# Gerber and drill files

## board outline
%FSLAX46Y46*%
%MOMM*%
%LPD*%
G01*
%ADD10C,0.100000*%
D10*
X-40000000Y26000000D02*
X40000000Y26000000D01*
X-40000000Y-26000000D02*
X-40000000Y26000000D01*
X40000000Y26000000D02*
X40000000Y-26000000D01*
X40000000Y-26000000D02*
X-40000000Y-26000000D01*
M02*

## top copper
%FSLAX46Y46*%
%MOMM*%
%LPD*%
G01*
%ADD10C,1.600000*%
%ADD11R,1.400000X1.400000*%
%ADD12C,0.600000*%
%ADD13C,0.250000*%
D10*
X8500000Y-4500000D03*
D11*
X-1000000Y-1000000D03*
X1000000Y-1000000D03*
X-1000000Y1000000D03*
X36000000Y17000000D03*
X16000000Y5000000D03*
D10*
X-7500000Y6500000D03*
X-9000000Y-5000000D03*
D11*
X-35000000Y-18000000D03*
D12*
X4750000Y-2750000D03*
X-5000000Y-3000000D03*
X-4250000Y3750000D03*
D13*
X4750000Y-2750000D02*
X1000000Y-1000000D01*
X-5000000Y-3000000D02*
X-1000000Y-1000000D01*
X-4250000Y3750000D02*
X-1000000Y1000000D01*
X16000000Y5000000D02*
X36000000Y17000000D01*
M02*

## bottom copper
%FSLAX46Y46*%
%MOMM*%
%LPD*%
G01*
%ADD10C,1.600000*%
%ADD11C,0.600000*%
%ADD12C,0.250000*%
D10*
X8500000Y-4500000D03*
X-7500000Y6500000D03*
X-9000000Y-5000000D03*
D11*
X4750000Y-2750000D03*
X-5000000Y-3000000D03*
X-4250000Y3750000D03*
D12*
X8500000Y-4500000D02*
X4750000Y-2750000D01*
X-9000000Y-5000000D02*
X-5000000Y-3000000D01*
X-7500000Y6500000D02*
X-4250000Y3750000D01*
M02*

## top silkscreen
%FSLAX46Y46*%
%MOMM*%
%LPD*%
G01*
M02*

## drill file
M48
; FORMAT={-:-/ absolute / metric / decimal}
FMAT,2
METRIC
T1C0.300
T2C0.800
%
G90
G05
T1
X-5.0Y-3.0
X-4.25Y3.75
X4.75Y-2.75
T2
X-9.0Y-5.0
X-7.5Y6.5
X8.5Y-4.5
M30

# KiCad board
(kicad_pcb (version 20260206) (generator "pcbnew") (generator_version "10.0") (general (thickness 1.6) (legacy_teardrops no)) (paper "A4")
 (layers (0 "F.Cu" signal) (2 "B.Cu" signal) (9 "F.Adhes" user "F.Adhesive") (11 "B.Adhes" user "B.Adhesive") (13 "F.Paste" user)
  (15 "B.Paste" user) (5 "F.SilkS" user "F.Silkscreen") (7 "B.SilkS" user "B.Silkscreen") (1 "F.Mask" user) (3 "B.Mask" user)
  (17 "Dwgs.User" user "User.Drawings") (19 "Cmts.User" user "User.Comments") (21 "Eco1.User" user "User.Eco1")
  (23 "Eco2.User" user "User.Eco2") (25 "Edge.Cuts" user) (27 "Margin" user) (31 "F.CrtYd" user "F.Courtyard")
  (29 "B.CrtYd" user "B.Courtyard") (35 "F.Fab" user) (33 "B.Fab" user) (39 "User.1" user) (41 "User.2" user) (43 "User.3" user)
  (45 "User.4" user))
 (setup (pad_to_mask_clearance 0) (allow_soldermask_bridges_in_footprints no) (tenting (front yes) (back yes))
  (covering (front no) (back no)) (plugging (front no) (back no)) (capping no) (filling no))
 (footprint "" (layer "F.Cu") (at 8.5 4.5)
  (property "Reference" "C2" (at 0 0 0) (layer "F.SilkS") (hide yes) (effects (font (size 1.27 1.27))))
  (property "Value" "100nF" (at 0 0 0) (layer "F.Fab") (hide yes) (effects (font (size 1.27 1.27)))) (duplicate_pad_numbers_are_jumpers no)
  (pad "1" thru_hole circle (at 0 0) (size 1.6 1.6) (drill 0.8) (layers "*.Cu" "*.Mask") (remove_unused_layers no) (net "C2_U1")))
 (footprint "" (layer "F.Cu") (at 0 0)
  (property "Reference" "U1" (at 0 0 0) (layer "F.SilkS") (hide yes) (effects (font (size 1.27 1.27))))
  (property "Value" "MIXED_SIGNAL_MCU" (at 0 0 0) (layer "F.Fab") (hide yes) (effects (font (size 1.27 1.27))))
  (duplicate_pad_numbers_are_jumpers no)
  (pad "1" smd rect (at -1 1) (size 1.4 1.4) (layers "F.Cu" "F.Mask" "F.Paste") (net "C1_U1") (thermal_bridge_angle 45))
  (pad "2" smd rect (at 1 1) (size 1.4 1.4) (layers "F.Cu" "F.Mask" "F.Paste") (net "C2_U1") (thermal_bridge_angle 45))
  (pad "3" smd rect (at -1 -1) (size 1.4 1.4) (layers "F.Cu" "F.Mask" "F.Paste") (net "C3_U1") (thermal_bridge_angle 45)))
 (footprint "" (layer "F.Cu") (at 36 -17)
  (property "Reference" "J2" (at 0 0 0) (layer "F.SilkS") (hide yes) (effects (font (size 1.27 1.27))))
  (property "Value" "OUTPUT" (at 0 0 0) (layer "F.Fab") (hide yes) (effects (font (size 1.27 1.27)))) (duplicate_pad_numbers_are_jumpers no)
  (pad "1" smd rect (at 0 0) (size 1.4 1.4) (layers "F.Cu" "F.Mask" "F.Paste") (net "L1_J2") (thermal_bridge_angle 45)))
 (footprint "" (layer "F.Cu") (at 16 -5)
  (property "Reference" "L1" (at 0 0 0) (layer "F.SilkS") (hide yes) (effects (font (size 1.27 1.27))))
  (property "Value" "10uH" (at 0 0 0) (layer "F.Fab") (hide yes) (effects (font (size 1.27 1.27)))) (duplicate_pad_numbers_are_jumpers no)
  (pad "1" smd rect (at 0 0) (size 1.4 1.4) (layers "F.Cu" "F.Mask" "F.Paste") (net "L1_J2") (thermal_bridge_angle 45)))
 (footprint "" (layer "F.Cu") (at -7.5 -6.5)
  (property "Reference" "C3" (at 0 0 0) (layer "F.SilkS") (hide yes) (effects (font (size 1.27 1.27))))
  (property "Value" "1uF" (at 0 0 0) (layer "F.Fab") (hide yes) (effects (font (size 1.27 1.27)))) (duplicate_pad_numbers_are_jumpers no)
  (pad "1" thru_hole circle (at 0 0) (size 1.6 1.6) (drill 0.8) (layers "*.Cu" "*.Mask") (remove_unused_layers no) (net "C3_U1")))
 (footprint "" (layer "F.Cu") (at -9 5)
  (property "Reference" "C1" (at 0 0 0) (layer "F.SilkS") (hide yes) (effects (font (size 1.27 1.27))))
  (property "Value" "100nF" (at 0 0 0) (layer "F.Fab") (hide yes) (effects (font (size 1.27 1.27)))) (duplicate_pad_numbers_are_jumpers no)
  (pad "1" thru_hole circle (at 0 0) (size 1.6 1.6) (drill 0.8) (layers "*.Cu" "*.Mask") (remove_unused_layers no) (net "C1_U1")))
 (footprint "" (layer "F.Cu") (at -35 18)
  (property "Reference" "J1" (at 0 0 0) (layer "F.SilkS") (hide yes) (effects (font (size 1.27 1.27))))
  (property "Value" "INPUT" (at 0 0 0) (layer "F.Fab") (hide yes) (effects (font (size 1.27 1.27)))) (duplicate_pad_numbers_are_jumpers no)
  (pad "1" smd rect (at 0 0) (size 1.4 1.4) (layers "F.Cu" "F.Mask" "F.Paste") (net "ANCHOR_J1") (thermal_bridge_angle 45)))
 (gr_line (start -40 -26) (end 40 -26) (stroke (width 0.1) (type default)) (layer "Edge.Cuts"))
 (gr_line (start -40 26) (end -40 -26) (stroke (width 0.1) (type default)) (layer "Edge.Cuts"))
 (gr_line (start 40 -26) (end 40 26) (stroke (width 0.1) (type default)) (layer "Edge.Cuts"))
 (gr_line (start 40 26) (end -40 26) (stroke (width 0.1) (type default)) (layer "Edge.Cuts"))
 (segment (start 4.75 2.75) (end 1 1) (width 0.25) (layer "F.Cu") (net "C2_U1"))
 (via (at 4.75 2.75) (size 0.6) (drill 0.3) (layers "F.Cu" "B.Cu") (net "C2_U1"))
 (segment (start 8.5 4.5) (end 4.75 2.75) (width 0.25) (layer "B.Cu") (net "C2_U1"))
 (segment (start -5 3) (end -1 1) (width 0.25) (layer "F.Cu") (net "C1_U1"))
 (via (at -5 3) (size 0.6) (drill 0.3) (layers "F.Cu" "B.Cu") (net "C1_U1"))
 (segment (start -9 5) (end -5 3) (width 0.25) (layer "B.Cu") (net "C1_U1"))
 (segment (start -4.25 -3.75) (end -1 -1) (width 0.25) (layer "F.Cu") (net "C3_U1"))
 (via (at -4.25 -3.75) (size 0.6) (drill 0.3) (layers "F.Cu" "B.Cu") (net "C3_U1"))
 (segment (start -7.5 -6.5) (end -4.25 -3.75) (width 0.25) (layer "B.Cu") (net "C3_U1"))
 (segment (start 16 -5) (end 36 -17) (width 0.25) (layer "F.Cu") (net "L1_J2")))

